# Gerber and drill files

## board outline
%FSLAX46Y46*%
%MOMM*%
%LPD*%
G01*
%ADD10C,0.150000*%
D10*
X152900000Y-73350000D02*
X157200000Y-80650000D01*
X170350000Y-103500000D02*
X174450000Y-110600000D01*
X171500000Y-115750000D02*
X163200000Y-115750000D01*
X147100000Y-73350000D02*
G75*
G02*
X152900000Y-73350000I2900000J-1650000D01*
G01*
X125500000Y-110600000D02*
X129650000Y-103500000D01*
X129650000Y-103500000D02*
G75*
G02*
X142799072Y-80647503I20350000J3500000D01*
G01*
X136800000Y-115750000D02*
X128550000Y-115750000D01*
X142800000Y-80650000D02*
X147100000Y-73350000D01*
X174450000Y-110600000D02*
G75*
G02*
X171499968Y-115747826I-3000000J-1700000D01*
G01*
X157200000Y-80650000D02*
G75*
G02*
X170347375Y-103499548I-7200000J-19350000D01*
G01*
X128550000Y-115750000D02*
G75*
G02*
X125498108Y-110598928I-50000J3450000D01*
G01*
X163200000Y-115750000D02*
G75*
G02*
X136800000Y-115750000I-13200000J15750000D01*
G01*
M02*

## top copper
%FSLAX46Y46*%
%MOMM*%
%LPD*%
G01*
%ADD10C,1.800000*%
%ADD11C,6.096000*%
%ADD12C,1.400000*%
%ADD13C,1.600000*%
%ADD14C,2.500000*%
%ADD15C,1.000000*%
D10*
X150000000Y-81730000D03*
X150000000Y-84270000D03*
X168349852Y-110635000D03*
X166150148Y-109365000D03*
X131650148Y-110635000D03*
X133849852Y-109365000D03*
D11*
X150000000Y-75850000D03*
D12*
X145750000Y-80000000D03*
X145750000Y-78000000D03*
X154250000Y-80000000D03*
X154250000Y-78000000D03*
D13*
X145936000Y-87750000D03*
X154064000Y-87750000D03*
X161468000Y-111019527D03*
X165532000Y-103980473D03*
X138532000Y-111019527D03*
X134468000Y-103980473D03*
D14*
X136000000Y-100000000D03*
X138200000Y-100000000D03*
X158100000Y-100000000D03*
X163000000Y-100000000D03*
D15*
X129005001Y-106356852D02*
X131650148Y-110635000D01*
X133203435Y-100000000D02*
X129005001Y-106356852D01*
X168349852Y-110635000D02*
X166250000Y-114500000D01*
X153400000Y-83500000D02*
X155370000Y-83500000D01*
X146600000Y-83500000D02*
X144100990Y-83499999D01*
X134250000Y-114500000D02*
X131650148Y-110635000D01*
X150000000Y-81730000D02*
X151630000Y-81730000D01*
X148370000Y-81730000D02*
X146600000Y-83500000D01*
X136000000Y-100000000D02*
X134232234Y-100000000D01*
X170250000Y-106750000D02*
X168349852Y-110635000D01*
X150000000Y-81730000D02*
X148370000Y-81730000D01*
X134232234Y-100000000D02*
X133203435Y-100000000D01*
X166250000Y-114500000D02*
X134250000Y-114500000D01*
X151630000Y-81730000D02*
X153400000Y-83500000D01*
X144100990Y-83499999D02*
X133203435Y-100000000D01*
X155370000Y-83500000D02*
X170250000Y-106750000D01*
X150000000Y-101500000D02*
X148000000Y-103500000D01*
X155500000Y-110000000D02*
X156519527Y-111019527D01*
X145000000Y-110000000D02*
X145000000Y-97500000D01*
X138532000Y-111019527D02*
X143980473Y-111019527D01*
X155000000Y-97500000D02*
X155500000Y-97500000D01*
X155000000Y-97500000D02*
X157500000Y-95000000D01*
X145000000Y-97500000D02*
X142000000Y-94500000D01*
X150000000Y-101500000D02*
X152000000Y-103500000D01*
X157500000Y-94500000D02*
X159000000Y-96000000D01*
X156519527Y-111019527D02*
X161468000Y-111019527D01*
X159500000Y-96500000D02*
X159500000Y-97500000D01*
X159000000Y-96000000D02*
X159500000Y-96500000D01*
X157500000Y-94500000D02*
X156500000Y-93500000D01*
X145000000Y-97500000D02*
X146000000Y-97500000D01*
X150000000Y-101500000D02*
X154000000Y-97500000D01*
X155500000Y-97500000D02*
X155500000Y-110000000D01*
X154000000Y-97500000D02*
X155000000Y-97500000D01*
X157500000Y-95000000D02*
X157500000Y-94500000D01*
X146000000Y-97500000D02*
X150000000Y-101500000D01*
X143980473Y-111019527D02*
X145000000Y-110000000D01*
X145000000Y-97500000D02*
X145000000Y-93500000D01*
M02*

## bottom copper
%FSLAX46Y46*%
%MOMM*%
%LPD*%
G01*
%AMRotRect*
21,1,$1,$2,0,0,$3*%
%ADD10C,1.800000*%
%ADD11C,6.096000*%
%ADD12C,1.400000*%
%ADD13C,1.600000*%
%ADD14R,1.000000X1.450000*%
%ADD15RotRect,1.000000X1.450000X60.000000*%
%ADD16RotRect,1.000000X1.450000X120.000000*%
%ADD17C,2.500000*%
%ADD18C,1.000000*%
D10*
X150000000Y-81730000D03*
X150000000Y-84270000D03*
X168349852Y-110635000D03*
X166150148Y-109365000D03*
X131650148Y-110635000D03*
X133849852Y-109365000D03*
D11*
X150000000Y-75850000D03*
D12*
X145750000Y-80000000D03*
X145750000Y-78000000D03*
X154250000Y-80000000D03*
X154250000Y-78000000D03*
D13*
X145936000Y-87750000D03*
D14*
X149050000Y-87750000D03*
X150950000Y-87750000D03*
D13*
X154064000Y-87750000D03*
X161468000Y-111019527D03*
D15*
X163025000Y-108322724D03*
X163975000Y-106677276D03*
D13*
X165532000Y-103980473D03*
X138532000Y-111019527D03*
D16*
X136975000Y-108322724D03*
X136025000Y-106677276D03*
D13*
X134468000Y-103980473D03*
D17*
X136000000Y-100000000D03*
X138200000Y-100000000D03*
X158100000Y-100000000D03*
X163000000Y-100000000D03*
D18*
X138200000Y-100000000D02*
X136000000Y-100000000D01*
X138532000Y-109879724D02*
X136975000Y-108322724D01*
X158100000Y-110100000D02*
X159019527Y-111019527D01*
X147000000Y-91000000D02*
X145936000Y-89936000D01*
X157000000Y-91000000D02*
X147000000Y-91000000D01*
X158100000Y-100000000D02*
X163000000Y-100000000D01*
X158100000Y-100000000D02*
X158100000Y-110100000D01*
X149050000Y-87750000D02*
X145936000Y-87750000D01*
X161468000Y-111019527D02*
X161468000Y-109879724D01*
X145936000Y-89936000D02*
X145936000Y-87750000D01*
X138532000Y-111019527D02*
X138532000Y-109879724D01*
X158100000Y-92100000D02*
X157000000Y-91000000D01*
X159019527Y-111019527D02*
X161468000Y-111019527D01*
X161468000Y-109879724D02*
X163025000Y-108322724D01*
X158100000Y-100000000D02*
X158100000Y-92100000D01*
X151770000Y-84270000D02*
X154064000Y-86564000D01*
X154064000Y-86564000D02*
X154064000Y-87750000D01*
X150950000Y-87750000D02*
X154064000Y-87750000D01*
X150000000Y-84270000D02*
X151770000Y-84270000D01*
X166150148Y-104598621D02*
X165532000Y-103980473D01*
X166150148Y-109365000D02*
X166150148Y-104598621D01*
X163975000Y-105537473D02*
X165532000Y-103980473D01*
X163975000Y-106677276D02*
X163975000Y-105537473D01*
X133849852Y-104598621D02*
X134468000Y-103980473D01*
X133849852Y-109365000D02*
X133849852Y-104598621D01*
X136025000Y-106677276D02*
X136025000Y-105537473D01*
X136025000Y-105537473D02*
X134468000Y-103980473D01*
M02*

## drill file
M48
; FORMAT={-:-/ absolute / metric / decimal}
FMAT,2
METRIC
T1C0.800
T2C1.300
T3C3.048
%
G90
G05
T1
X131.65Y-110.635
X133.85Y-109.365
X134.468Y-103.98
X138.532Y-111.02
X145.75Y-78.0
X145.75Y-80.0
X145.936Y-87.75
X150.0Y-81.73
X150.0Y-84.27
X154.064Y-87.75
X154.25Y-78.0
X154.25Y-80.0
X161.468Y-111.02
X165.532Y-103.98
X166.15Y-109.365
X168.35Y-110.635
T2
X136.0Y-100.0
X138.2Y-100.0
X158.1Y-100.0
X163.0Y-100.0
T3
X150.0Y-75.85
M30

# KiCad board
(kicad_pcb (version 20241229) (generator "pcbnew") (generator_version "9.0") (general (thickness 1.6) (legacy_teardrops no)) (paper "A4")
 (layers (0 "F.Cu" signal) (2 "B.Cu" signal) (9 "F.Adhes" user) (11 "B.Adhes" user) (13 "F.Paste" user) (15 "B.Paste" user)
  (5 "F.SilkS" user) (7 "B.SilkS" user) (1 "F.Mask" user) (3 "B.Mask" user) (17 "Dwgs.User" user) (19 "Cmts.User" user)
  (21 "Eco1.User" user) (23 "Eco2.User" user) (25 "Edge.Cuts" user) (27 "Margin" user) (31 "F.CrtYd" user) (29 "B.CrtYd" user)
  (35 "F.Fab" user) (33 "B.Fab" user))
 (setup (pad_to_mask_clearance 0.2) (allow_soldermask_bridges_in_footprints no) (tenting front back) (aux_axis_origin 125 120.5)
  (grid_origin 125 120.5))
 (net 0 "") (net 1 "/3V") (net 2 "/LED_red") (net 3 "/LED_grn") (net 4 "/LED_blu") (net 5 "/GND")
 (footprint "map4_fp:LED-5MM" (layer "F.Cu") (at 150 83 -90)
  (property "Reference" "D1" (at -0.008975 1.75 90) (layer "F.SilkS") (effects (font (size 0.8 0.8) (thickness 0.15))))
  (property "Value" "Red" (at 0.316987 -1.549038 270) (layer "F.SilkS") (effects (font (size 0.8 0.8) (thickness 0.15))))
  (pad "1" thru_hole circle (at -1.27 0 270) (size 1.8 1.8) (drill 0.8) (layers "*.Cu" "*.Mask" "F.SilkS") (remove_unused_layers no)
   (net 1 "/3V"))
  (pad "2" thru_hole circle (at 1.27 0 270) (size 1.8 1.8) (drill 0.8) (layers "*.Cu" "*.Mask" "F.SilkS") (remove_unused_layers no)
   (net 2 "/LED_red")))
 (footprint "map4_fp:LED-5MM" (layer "F.Cu") (at 167.25 110 150)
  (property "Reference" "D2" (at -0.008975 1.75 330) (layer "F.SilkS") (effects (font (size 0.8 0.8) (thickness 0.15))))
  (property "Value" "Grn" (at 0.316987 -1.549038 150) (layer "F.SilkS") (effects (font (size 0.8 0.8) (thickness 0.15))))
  (pad "1" thru_hole circle (at -1.27 0 150) (size 1.8 1.8) (drill 0.8) (layers "*.Cu" "*.Mask" "F.SilkS") (remove_unused_layers no)
   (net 1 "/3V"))
  (pad "2" thru_hole circle (at 1.27 0 150) (size 1.8 1.8) (drill 0.8) (layers "*.Cu" "*.Mask" "F.SilkS") (remove_unused_layers no)
   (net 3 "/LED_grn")))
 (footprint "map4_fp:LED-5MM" (layer "F.Cu") (at 132.75 110 30)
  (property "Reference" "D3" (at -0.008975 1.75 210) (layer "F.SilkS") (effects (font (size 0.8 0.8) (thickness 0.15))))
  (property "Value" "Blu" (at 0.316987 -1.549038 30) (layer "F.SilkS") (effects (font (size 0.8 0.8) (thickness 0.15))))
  (pad "1" thru_hole circle (at -1.27 0 30) (size 1.8 1.8) (drill 0.8) (layers "*.Cu" "*.Mask" "F.SilkS") (remove_unused_layers no)
   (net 1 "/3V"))
  (pad "2" thru_hole circle (at 1.27 0 30) (size 1.8 1.8) (drill 0.8) (layers "*.Cu" "*.Mask" "F.SilkS") (remove_unused_layers no)
   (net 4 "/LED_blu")))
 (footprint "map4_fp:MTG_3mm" (layer "F.Cu") (at 150 75.85)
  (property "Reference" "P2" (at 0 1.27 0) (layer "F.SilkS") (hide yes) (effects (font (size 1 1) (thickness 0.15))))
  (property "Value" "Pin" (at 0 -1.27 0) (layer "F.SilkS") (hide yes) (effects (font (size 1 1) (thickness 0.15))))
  (pad "1" thru_hole circle (at 0 0) (size 6.096 6.096) (drill 3.048) (layers "*.Cu" "*.Mask" "F.SilkS") (remove_unused_layers no)))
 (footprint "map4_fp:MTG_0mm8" (layer "F.Cu") (at 145.75 80)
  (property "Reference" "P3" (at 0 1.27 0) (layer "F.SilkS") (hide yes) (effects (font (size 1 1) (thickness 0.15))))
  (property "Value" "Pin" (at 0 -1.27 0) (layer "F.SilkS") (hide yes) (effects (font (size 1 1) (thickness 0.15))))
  (pad "1" thru_hole circle (at 0 0) (size 1.4 1.4) (drill 0.8) (layers "*.Cu" "*.Mask" "F.SilkS") (remove_unused_layers no)))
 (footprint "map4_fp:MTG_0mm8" (layer "F.Cu") (at 145.75 78)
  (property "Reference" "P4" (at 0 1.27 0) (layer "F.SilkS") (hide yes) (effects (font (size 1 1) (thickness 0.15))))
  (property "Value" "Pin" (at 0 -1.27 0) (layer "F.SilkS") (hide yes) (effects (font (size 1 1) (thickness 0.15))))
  (pad "1" thru_hole circle (at 0 0) (size 1.4 1.4) (drill 0.8) (layers "*.Cu" "*.Mask" "F.SilkS") (remove_unused_layers no)))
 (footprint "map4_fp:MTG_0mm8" (layer "F.Cu") (at 154.25 80)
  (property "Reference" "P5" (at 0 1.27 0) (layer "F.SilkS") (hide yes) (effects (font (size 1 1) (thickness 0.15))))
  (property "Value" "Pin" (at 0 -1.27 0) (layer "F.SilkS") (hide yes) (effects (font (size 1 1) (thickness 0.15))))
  (pad "1" thru_hole circle (at 0 0) (size 1.4 1.4) (drill 0.8) (layers "*.Cu" "*.Mask" "F.SilkS") (remove_unused_layers no)))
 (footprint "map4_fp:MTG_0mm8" (layer "F.Cu") (at 154.25 78)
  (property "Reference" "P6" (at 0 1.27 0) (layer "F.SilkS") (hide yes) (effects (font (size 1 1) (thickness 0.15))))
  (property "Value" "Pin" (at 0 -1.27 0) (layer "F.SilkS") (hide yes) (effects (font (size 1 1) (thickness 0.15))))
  (pad "1" thru_hole circle (at 0 0) (size 1.4 1.4) (drill 0.8) (layers "*.Cu" "*.Mask" "F.SilkS") (remove_unused_layers no)))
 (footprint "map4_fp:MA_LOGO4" (layer "F.Cu") (at 150 97.5)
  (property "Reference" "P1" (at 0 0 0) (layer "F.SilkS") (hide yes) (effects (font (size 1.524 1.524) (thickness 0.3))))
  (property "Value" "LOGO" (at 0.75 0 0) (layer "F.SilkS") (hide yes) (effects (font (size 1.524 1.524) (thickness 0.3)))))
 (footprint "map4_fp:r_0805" (layer "B.Cu") (at 150 87.75)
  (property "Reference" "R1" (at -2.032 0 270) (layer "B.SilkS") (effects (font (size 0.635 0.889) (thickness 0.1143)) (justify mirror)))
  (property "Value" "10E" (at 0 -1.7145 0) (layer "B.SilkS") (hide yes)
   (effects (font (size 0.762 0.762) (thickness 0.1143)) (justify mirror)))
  (pad "1" thru_hole circle (at -4.064 0) (size 1.6 1.6) (drill 0.8) (layers "*.Cu" "*.Mask" "B.SilkS") (remove_unused_layers no)
   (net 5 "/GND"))
  (pad "1" smd rect (at -0.95 0) (size 1 1.45) (layers "B.Cu" "B.Mask" "B.Paste") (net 5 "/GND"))
  (pad "2" smd rect (at 0.95 0) (size 1 1.45) (layers "B.Cu" "B.Mask" "B.Paste") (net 2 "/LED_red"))
  (pad "2" thru_hole circle (at 4.064 0) (size 1.6 1.6) (drill 0.8) (layers "*.Cu" "*.Mask" "B.SilkS") (remove_unused_layers no)
   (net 2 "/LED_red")))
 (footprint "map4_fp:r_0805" (layer "B.Cu") (at 163.5 107.5 60)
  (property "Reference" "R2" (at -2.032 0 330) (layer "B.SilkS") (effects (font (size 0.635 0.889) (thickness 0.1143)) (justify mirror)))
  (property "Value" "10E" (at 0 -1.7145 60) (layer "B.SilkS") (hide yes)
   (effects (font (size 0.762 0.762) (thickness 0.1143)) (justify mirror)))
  (pad "1" thru_hole circle (at -4.064 0 60) (size 1.6 1.6) (drill 0.8) (layers "*.Cu" "*.Mask" "B.SilkS") (remove_unused_layers no)
   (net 5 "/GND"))
  (pad "1" smd rect (at -0.95 0 60) (size 1 1.45) (layers "B.Cu" "B.Mask" "B.Paste") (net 5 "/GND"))
  (pad "2" smd rect (at 0.95 0 60) (size 1 1.45) (layers "B.Cu" "B.Mask" "B.Paste") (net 3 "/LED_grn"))
  (pad "2" thru_hole circle (at 4.064 0 60) (size 1.6 1.6) (drill 0.8) (layers "*.Cu" "*.Mask" "B.SilkS") (remove_unused_layers no)
   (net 3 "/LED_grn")))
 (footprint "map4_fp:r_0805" (layer "B.Cu") (at 136.5 107.5 120)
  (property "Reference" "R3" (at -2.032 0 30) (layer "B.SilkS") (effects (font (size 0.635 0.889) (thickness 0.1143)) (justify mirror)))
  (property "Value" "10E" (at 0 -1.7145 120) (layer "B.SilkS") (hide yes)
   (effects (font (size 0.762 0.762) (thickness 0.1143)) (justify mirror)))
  (pad "1" thru_hole circle (at -4.064 0 120) (size 1.6 1.6) (drill 0.8) (layers "*.Cu" "*.Mask" "B.SilkS") (remove_unused_layers no)
   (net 5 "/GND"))
  (pad "1" smd rect (at -0.95 0 120) (size 1 1.45) (layers "B.Cu" "B.Mask" "B.Paste") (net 5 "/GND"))
  (pad "2" smd rect (at 0.95 0 120) (size 1 1.45) (layers "B.Cu" "B.Mask" "B.Paste") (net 4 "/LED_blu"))
  (pad "2" thru_hole circle (at 4.064 0 120) (size 1.6 1.6) (drill 0.8) (layers "*.Cu" "*.Mask" "B.SilkS") (remove_unused_layers no)
   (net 4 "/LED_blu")))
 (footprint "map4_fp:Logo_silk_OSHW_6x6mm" (layer "B.Cu") (at 150 107.5 180)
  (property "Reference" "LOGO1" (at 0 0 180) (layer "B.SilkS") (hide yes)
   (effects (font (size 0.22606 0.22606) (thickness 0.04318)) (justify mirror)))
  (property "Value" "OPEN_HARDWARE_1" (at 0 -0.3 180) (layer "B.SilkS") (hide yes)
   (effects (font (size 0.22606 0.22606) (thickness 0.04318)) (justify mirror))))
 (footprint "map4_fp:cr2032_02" (layer "B.Cu") (at 150 100 90)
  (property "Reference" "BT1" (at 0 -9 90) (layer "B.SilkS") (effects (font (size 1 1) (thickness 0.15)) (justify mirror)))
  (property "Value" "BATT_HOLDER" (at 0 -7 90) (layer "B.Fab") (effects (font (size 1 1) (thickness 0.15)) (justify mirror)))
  (pad "1" thru_hole circle (at 0 -14 90) (size 2.5 2.5) (drill 1.3) (layers "*.Cu" "*.Mask" "B.SilkS") (remove_unused_layers no)
   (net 1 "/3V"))
  (pad "1" thru_hole circle (at 0 -11.8 90) (size 2.5 2.5) (drill 1.3) (layers "*.Cu" "*.Mask" "B.SilkS") (remove_unused_layers no)
   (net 1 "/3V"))
  (pad "2" thru_hole circle (at 0 8.1 90) (size 2.5 2.5) (drill 1.3) (layers "*.Cu" "*.Mask" "B.SilkS") (remove_unused_layers no)
   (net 5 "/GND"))
  (pad "2" thru_hole circle (at 0 13 90) (size 2.5 2.5) (drill 1.3) (layers "*.Cu" "*.Mask" "B.SilkS") (remove_unused_layers no)
   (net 5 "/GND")))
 (gr_line (start 152.9 73.35) (end 157.2 80.65) (stroke (width 0.15) (type solid)) (layer "Edge.Cuts"))
 (gr_line (start 170.35 103.5) (end 174.45 110.6) (stroke (width 0.15) (type solid)) (layer "Edge.Cuts"))
 (gr_line (start 171.5 115.75) (end 163.2 115.75) (stroke (width 0.15) (type solid)) (layer "Edge.Cuts"))
 (gr_arc (start 147.1 73.35) (mid 150 71.66346) (end 152.9 73.35) (stroke (width 0.15) (type solid)) (layer "Edge.Cuts"))
 (gr_line (start 125.5 110.6) (end 129.65 103.5) (stroke (width 0.15) (type solid)) (layer "Edge.Cuts"))
 (gr_arc (start 129.65 103.5) (mid 132.102443 89.701945) (end 142.799072 80.647503) (stroke (width 0.15) (type solid)) (layer "Edge.Cuts"))
 (gr_line (start 136.8 115.75) (end 128.55 115.75) (stroke (width 0.15) (type solid)) (layer "Edge.Cuts"))
 (gr_line (start 142.8 80.65) (end 147.1 73.35) (stroke (width 0.15) (type solid)) (layer "Edge.Cuts"))
 (gr_arc (start 174.45 110.6) (mid 174.441756 114.014467) (end 171.499968 115.747826) (stroke (width 0.15) (type solid)) (layer "Edge.Cuts"))
 (gr_arc (start 157.2 80.65) (mid 167.895249 89.703274) (end 170.347375 103.499548) (stroke (width 0.15) (type solid)) (layer "Edge.Cuts"))
 (gr_arc (start 128.55 115.75) (mid 125.531532 114.058749) (end 125.498108 110.598928) (stroke (width 0.15) (type solid))
  (layer "Edge.Cuts"))
 (gr_arc (start 163.2 115.75) (mid 150 120.55) (end 136.8 115.75) (stroke (width 0.15) (type solid)) (layer "Edge.Cuts"))
 (segment (start 129.005001 106.356852) (end 131.650148 110.635) (width 1) (layer "F.Cu") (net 1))
 (segment (start 133.203435 100) (end 129.005001 106.356852) (width 1) (layer "F.Cu") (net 1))
 (segment (start 168.349852 110.635) (end 166.25 114.5) (width 1) (layer "F.Cu") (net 1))
 (segment (start 153.4 83.5) (end 155.37 83.5) (width 1) (layer "F.Cu") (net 1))
 (segment (start 146.6 83.5) (end 144.10099 83.499999) (width 1) (layer "F.Cu") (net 1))
 (segment (start 134.25 114.5) (end 131.650148 110.635) (width 1) (layer "F.Cu") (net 1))
 (segment (start 150 81.73) (end 151.63 81.73) (width 1) (layer "F.Cu") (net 1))
 (segment (start 148.37 81.73) (end 146.6 83.5) (width 1) (layer "F.Cu") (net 1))
 (segment (start 136 100) (end 134.232234 100) (width 1) (layer "F.Cu") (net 1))
 (segment (start 170.25 106.75) (end 168.349852 110.635) (width 1) (layer "F.Cu") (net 1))
 (segment (start 150 81.73) (end 148.37 81.73) (width 1) (layer "F.Cu") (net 1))
 (segment (start 134.232234 100) (end 133.203435 100) (width 1) (layer "F.Cu") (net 1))
 (segment (start 166.25 114.5) (end 134.25 114.5) (width 1) (layer "F.Cu") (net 1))
 (segment (start 151.63 81.73) (end 153.4 83.5) (width 1) (layer "F.Cu") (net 1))
 (segment (start 144.10099 83.499999) (end 133.203435 100) (width 1) (layer "F.Cu") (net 1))
 (segment (start 155.37 83.5) (end 170.25 106.75) (width 1) (layer "F.Cu") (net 1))
 (segment (start 138.2 100) (end 136 100) (width 1) (layer "B.Cu") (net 1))
 (segment (start 150 101.5) (end 148 103.5) (width 1) (layer "F.Cu") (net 5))
 (segment (start 155.5 110) (end 156.519527 111.019527) (width 1) (layer "F.Cu") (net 5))
 (segment (start 145 110) (end 145 97.5) (width 1) (layer "F.Cu") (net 5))
 (segment (start 138.532 111.019527) (end 143.980473 111.019527) (width 1) (layer "F.Cu") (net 5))
 (segment (start 155 97.5) (end 155.5 97.5) (width 1) (layer "F.Cu") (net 5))
 (segment (start 155 97.5) (end 157.5 95) (width 1) (layer "F.Cu") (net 5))
 (segment (start 145 97.5) (end 142 94.5) (width 1) (layer "F.Cu") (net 5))
 (segment (start 150 101.5) (end 152 103.5) (width 1) (layer "F.Cu") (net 5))
 (segment (start 157.5 94.5) (end 159 96) (width 1) (layer "F.Cu") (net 5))
 (segment (start 156.519527 111.019527) (end 161.468 111.019527) (width 1) (layer "F.Cu") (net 5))
 (segment (start 159.5 96.5) (end 159.5 97.5) (width 1) (layer "F.Cu") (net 5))
 (segment (start 159 96) (end 159.5 96.5) (width 1) (layer "F.Cu") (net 5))
 (segment (start 157.5 94.5) (end 156.5 93.5) (width 1) (layer "F.Cu") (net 5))
 (segment (start 145 97.5) (end 146 97.5) (width 1) (layer "F.Cu") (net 5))
 (segment (start 150 101.5) (end 154 97.5) (width 1) (layer "F.Cu") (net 5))
 (segment (start 155.5 97.5) (end 155.5 110) (width 1) (layer "F.Cu") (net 5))
 (segment (start 154 97.5) (end 155 97.5) (width 1) (layer "F.Cu") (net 5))
 (segment (start 157.5 95) (end 157.5 94.5) (width 1) (layer "F.Cu") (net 5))
 (segment (start 146 97.5) (end 150 101.5) (width 1) (layer "F.Cu") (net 5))
 (segment (start 143.980473 111.019527) (end 145 110) (width 1) (layer "F.Cu") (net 5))
 (segment (start 145 97.5) (end 145 93.5) (width 1) (layer "F.Cu") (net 5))
 (segment (start 138.532 109.879724) (end 136.975 108.322724) (width 1) (layer "B.Cu") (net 5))
 (segment (start 158.1 110.1) (end 159.019527 111.019527) (width 1) (layer "B.Cu") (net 5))
 (segment (start 147 91) (end 145.936 89.936) (width 1) (layer "B.Cu") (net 5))
 (segment (start 157 91) (end 147 91) (width 1) (layer "B.Cu") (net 5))
 (segment (start 158.1 100) (end 163 100) (width 1) (layer "B.Cu") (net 5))
 (segment (start 158.1 100) (end 158.1 110.1) (width 1) (layer "B.Cu") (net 5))
 (segment (start 149.05 87.75) (end 145.936 87.75) (width 1) (layer "B.Cu") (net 5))
 (segment (start 161.468 111.019527) (end 161.468 109.879724) (width 1) (layer "B.Cu") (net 5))
 (segment (start 145.936 89.936) (end 145.936 87.75) (width 1) (layer "B.Cu") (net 5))
 (segment (start 138.532 111.019527) (end 138.532 109.879724) (width 1) (layer "B.Cu") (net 5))
 (segment (start 158.1 92.1) (end 157 91) (width 1) (layer "B.Cu") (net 5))
 (segment (start 159.019527 111.019527) (end 161.468 111.019527) (width 1) (layer "B.Cu") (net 5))
 (segment (start 161.468 109.879724) (end 163.025 108.322724) (width 1) (layer "B.Cu") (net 5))
 (segment (start 158.1 100) (end 158.1 92.1) (width 1) (layer "B.Cu") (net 5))
 (segment (start 151.77 84.27) (end 154.064 86.564) (width 1) (layer "B.Cu") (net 2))
 (segment (start 154.064 86.564) (end 154.064 87.75) (width 1) (layer "B.Cu") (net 2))
 (segment (start 150.95 87.75) (end 154.064 87.75) (width 1) (layer "B.Cu") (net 2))
 (segment (start 150 84.27) (end 151.77 84.27) (width 1) (layer "B.Cu") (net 2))
 (segment (start 166.150148 104.598621) (end 165.532 103.980473) (width 1) (layer "B.Cu") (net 3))
 (segment (start 166.150148 109.365) (end 166.150148 104.598621) (width 1) (layer "B.Cu") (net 3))
 (segment (start 163.975 105.537473) (end 165.532 103.980473) (width 1) (layer "B.Cu") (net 3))
 (segment (start 163.975 106.677276) (end 163.975 105.537473) (width 1) (layer "B.Cu") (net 3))
 (segment (start 133.849852 104.598621) (end 134.468 103.980473) (width 1) (layer "B.Cu") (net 4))
 (segment (start 133.849852 109.365) (end 133.849852 104.598621) (width 1) (layer "B.Cu") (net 4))
 (segment (start 136.025 106.677276) (end 136.025 105.537473) (width 1) (layer "B.Cu") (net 4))
 (segment (start 136.025 105.537473) (end 134.468 103.980473) (width 1) (layer "B.Cu") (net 4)))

